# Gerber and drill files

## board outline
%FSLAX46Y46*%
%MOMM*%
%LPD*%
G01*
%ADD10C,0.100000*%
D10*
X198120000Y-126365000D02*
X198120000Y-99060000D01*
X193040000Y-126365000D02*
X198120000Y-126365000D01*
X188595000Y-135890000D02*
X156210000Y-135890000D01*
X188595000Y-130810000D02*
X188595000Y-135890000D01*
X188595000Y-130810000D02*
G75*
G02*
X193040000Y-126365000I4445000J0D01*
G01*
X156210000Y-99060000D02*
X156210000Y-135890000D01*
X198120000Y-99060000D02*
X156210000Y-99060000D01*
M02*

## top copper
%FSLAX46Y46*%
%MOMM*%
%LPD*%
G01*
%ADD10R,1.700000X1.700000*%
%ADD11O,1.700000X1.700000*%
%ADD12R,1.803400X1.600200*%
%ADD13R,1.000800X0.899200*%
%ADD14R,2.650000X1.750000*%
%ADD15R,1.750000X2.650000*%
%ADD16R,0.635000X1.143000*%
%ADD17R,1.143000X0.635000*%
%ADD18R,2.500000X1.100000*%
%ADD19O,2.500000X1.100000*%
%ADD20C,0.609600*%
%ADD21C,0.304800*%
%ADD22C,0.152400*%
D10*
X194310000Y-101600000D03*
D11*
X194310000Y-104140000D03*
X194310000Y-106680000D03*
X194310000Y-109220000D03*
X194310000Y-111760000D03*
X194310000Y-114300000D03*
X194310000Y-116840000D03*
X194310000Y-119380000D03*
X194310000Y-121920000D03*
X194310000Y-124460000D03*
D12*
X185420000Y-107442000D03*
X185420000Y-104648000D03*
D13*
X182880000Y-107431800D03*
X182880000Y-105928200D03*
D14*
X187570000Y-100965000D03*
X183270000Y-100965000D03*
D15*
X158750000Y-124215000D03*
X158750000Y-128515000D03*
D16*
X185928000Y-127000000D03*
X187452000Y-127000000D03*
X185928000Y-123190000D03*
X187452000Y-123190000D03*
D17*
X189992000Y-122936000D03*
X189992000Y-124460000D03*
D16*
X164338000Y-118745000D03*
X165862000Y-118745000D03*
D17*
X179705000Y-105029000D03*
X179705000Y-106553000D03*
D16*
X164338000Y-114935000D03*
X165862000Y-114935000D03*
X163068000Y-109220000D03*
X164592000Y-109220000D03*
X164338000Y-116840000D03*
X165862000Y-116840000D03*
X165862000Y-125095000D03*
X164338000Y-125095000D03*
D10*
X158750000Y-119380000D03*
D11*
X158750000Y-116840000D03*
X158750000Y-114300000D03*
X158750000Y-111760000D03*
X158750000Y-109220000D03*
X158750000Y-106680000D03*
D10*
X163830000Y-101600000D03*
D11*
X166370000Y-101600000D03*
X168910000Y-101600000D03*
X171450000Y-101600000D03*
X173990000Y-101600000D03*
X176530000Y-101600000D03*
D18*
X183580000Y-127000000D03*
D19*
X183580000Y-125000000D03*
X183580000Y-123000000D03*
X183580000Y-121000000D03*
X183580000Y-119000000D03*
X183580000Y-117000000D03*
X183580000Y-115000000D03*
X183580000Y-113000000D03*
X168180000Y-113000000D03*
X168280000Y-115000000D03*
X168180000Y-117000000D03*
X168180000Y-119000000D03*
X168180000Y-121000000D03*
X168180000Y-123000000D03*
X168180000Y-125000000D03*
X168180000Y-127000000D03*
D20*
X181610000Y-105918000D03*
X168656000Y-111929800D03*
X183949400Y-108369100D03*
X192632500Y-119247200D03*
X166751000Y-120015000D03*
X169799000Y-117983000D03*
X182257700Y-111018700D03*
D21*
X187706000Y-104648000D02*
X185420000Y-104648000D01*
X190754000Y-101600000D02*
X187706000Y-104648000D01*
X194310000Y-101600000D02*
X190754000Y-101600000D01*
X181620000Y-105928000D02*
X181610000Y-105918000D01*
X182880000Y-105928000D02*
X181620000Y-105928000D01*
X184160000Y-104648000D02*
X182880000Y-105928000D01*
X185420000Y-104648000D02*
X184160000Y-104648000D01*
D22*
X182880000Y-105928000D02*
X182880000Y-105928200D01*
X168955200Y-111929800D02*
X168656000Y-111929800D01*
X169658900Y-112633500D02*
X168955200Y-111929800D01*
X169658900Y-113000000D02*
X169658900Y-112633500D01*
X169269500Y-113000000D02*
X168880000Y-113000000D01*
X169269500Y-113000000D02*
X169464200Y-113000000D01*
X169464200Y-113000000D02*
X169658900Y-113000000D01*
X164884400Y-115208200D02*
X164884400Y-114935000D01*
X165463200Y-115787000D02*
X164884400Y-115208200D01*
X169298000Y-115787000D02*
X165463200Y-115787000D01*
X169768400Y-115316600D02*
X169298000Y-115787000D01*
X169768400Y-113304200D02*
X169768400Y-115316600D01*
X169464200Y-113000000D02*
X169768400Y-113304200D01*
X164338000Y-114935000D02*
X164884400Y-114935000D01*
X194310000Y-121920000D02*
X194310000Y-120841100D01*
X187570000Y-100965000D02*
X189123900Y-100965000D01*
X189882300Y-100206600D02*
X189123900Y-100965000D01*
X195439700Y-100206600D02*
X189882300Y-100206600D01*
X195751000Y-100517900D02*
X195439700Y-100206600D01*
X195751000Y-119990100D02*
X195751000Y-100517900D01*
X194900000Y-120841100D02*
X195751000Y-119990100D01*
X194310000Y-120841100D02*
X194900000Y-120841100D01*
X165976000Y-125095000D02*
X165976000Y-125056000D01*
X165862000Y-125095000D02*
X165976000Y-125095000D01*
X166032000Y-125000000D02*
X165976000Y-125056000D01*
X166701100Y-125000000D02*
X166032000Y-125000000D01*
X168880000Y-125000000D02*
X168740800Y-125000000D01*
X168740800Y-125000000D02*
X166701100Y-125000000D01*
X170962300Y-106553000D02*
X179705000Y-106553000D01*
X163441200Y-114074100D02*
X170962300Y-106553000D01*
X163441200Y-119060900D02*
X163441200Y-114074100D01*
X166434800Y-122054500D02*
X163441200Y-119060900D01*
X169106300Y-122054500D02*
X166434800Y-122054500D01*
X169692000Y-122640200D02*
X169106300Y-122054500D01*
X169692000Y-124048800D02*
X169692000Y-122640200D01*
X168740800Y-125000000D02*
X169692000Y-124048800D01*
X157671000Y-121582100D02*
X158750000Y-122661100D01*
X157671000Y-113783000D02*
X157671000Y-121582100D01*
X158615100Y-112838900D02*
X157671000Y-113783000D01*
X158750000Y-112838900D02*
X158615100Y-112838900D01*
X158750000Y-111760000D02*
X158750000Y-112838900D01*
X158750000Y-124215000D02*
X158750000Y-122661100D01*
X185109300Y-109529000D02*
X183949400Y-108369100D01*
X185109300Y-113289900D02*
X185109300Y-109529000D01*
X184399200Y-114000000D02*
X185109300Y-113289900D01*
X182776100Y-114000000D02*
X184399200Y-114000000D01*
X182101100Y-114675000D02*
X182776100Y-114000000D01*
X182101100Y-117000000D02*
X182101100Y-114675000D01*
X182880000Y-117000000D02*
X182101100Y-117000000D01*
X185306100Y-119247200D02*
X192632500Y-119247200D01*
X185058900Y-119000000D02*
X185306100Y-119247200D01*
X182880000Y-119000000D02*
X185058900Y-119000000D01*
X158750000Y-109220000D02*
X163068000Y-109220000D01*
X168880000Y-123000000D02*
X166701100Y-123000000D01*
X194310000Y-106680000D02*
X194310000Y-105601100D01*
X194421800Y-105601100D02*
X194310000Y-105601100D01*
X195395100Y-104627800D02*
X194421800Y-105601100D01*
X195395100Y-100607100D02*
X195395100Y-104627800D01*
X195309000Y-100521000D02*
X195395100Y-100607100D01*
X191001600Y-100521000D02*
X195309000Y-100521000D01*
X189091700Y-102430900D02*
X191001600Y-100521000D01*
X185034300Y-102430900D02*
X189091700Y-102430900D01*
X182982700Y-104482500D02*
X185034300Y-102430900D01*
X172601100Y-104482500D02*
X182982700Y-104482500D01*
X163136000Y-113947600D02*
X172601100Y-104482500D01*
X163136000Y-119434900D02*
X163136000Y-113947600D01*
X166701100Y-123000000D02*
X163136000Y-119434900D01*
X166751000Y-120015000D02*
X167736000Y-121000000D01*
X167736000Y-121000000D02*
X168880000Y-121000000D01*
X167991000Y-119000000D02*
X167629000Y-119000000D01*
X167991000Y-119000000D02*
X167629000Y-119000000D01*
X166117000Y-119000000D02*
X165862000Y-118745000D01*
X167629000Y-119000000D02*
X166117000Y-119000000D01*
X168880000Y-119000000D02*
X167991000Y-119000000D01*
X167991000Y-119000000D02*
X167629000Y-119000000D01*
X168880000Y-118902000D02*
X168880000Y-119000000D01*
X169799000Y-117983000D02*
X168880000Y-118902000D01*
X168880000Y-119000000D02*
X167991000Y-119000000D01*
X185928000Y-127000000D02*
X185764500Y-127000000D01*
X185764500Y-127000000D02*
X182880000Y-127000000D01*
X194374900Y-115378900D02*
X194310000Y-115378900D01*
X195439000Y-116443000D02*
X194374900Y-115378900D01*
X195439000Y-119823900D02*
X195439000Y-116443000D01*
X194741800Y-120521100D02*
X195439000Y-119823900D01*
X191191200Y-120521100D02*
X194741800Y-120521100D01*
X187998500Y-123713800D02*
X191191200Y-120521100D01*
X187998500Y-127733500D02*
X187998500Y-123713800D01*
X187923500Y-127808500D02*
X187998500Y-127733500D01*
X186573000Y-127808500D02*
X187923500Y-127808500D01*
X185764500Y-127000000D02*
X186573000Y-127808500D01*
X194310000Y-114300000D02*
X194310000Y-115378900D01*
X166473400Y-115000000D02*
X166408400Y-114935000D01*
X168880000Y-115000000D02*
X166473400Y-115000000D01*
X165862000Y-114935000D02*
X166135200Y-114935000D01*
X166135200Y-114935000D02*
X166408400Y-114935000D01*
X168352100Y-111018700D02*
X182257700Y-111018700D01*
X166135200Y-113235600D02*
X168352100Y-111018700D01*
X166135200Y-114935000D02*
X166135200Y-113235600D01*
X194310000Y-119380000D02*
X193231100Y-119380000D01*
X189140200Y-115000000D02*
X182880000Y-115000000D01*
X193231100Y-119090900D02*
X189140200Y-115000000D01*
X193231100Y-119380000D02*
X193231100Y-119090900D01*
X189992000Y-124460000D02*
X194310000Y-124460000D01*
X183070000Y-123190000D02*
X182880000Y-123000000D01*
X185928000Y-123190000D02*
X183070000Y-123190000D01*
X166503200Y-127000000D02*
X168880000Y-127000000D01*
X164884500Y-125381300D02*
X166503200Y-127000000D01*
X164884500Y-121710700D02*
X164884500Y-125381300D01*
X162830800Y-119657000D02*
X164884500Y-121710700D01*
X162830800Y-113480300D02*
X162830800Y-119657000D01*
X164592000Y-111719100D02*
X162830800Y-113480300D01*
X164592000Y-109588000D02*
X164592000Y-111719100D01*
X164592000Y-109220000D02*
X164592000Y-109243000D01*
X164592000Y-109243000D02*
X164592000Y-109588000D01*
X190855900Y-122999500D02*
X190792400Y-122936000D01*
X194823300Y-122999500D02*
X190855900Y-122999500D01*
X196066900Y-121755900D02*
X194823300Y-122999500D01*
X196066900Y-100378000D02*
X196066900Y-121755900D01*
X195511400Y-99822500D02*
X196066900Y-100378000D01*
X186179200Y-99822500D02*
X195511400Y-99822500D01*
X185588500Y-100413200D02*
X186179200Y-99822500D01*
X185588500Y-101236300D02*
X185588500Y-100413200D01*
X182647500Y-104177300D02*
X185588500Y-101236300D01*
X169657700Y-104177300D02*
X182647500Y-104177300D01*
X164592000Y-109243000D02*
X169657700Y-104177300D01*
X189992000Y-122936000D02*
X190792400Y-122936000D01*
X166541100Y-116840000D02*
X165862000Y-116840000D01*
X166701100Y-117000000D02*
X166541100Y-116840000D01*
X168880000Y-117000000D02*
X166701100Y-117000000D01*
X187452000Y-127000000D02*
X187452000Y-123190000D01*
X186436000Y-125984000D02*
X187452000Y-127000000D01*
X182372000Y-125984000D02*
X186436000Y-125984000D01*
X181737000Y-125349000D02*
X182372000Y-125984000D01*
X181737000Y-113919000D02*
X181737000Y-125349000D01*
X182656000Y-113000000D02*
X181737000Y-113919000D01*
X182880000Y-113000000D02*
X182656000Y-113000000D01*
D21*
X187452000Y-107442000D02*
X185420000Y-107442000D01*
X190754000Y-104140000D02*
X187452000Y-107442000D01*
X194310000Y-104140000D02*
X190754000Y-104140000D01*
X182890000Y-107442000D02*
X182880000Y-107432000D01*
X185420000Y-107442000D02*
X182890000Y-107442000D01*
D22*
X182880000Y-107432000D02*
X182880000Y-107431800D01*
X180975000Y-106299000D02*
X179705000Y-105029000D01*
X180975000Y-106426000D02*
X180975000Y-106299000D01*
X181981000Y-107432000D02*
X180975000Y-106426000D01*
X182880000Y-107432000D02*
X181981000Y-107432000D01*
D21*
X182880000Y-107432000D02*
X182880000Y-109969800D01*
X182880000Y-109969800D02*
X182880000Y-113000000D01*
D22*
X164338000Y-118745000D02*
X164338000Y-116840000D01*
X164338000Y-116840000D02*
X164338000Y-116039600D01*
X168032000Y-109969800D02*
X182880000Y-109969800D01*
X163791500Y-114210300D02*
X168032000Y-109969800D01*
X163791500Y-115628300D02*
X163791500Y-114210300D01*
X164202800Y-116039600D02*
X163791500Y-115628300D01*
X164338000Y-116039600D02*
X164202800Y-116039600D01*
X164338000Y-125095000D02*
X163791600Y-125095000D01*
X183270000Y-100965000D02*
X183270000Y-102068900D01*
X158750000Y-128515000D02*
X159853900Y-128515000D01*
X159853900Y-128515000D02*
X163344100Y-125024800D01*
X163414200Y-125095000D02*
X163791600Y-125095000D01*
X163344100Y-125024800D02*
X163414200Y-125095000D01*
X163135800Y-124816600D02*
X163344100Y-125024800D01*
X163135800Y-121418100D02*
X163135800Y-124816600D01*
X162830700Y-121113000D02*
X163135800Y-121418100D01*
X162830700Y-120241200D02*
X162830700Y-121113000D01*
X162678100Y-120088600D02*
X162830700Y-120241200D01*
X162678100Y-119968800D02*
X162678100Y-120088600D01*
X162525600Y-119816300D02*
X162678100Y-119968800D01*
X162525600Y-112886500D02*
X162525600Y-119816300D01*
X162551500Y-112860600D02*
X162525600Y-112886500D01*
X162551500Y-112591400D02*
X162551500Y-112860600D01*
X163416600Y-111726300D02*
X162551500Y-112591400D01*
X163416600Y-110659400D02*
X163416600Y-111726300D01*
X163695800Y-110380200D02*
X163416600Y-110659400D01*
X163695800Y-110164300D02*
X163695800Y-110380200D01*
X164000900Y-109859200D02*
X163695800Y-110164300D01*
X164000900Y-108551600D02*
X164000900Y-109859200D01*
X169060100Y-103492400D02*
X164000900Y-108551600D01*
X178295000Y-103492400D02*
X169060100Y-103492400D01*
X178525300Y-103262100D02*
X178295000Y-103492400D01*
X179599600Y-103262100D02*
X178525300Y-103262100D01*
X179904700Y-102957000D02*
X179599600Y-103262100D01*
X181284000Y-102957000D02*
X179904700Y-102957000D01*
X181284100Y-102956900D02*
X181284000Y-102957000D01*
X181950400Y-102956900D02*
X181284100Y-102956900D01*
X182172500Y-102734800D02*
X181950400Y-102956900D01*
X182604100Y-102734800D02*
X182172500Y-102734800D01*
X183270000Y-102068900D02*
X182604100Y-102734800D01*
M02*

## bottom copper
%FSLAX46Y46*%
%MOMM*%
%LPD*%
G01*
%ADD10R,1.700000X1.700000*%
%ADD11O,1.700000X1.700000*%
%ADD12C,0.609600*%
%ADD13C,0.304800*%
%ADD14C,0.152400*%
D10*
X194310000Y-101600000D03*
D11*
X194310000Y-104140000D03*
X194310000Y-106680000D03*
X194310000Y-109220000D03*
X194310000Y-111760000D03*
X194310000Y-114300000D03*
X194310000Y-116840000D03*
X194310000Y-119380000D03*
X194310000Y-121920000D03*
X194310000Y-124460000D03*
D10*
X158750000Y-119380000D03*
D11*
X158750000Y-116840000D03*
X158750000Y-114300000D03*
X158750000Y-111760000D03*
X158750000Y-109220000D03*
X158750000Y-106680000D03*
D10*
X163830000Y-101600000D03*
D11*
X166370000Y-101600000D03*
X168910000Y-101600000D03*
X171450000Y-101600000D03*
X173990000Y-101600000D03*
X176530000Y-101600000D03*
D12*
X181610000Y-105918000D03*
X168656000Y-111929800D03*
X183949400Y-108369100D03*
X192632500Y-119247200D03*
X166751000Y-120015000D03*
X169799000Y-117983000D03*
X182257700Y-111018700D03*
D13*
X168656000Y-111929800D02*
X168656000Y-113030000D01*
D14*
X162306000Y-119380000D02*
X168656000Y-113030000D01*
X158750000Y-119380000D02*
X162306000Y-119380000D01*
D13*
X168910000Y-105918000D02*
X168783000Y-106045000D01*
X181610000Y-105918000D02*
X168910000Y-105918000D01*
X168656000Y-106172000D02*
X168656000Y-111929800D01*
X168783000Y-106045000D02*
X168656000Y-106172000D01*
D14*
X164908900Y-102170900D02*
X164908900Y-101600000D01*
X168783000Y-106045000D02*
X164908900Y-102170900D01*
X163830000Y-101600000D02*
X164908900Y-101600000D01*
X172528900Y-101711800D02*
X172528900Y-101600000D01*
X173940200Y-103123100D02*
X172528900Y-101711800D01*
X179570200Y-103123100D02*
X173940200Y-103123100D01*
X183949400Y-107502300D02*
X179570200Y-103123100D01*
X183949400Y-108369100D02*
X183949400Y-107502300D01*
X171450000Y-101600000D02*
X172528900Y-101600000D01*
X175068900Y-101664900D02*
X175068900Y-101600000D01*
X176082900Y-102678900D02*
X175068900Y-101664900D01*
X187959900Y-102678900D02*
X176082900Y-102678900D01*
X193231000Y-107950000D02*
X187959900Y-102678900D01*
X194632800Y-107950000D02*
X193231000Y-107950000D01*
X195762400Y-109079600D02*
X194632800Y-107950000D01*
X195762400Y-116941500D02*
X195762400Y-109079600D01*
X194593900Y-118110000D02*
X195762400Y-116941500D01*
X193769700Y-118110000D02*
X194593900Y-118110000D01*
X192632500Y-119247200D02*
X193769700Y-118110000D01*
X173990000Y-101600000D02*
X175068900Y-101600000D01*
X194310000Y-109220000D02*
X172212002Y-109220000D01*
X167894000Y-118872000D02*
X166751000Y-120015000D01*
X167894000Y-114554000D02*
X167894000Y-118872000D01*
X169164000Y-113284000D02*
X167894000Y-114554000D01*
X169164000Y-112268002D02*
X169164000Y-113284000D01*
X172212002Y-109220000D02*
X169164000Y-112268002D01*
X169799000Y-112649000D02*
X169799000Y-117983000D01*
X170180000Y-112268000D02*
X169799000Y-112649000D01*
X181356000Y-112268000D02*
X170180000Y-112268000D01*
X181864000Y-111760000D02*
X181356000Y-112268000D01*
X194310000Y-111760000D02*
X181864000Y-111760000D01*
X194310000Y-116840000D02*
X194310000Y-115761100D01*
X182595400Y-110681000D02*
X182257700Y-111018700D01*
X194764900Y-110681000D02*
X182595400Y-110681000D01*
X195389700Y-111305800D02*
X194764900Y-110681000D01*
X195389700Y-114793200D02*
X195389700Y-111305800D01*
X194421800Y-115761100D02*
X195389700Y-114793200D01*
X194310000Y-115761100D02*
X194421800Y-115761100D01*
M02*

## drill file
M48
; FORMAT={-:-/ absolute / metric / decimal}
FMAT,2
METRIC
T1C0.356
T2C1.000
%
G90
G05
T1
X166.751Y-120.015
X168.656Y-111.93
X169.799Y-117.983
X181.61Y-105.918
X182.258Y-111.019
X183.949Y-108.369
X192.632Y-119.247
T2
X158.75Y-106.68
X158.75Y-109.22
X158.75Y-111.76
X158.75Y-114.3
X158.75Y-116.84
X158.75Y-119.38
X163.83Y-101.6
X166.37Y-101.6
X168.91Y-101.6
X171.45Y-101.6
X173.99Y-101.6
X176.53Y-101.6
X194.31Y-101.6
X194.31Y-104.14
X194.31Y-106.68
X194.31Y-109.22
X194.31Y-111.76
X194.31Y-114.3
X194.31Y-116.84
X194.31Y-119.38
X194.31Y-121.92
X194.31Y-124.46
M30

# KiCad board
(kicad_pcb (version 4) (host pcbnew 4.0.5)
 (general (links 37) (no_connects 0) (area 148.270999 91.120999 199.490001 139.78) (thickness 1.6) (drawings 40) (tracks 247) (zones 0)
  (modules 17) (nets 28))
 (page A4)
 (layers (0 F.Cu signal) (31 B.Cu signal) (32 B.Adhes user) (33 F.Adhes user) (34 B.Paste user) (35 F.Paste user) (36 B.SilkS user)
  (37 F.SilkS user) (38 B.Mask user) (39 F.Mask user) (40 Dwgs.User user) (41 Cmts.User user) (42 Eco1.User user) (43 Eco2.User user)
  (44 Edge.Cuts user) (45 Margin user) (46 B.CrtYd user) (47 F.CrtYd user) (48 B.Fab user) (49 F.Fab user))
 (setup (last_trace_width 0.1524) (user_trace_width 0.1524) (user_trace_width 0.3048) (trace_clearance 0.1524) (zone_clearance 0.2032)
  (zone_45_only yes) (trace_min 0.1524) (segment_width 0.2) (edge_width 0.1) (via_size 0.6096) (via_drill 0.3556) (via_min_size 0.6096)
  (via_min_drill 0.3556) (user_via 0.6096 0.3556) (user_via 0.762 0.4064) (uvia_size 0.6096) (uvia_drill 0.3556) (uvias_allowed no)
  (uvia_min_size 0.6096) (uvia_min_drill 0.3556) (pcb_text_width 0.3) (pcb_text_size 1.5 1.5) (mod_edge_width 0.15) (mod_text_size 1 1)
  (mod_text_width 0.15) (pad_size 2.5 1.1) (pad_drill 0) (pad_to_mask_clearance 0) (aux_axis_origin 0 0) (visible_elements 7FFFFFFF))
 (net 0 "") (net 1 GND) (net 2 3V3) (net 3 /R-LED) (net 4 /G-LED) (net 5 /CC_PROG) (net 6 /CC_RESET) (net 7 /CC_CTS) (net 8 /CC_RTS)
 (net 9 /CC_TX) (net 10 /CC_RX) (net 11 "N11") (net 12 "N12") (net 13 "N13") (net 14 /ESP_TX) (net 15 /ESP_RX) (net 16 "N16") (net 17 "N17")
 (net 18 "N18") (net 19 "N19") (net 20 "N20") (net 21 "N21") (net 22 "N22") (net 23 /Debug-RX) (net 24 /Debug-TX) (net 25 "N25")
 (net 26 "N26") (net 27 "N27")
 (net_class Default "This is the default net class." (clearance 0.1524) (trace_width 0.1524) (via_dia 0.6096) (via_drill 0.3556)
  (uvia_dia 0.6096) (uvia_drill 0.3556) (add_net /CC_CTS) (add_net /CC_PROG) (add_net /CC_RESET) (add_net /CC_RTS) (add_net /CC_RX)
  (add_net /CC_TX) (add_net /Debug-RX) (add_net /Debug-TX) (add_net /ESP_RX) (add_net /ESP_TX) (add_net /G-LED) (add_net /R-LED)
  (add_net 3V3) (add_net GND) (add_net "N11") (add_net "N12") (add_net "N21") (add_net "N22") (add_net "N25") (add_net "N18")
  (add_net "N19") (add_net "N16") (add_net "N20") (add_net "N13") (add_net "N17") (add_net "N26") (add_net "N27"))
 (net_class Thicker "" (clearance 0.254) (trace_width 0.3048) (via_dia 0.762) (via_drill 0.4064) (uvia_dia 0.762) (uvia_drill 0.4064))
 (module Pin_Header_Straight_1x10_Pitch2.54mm (layer B.Cu) (at 194.31 101.6 180)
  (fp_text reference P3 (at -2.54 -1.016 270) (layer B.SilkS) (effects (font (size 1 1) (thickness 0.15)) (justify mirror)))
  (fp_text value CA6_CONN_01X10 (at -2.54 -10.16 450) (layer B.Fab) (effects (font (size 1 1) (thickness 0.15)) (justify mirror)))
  (pad 1 thru_hole rect (at 0 0 180) (size 1.7 1.7) (drill 1) (layers *.Cu *.Mask) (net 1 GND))
  (pad 2 thru_hole oval (at 0 -2.54 180) (size 1.7 1.7) (drill 1) (layers *.Cu *.Mask) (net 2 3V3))
  (pad 3 thru_hole oval (at 0 -5.08 180) (size 1.7 1.7) (drill 1) (layers *.Cu *.Mask) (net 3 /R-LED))
  (pad 4 thru_hole oval (at 0 -7.62 180) (size 1.7 1.7) (drill 1) (layers *.Cu *.Mask) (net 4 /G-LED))
  (pad 5 thru_hole oval (at 0 -10.16 180) (size 1.7 1.7) (drill 1) (layers *.Cu *.Mask) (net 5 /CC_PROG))
  (pad 6 thru_hole oval (at 0 -12.7 180) (size 1.7 1.7) (drill 1) (layers *.Cu *.Mask) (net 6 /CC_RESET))
  (pad 7 thru_hole oval (at 0 -15.24 180) (size 1.7 1.7) (drill 1) (layers *.Cu *.Mask) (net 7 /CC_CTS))
  (pad 8 thru_hole oval (at 0 -17.78 180) (size 1.7 1.7) (drill 1) (layers *.Cu *.Mask) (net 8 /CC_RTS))
  (pad 9 thru_hole oval (at 0 -20.32 180) (size 1.7 1.7) (drill 1) (layers *.Cu *.Mask) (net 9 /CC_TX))
  (pad 10 thru_hole oval (at 0 -22.86 180) (size 1.7 1.7) (drill 1) (layers *.Cu *.Mask) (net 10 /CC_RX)))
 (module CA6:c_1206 (layer F.Cu) (at 185.42 106.045 270)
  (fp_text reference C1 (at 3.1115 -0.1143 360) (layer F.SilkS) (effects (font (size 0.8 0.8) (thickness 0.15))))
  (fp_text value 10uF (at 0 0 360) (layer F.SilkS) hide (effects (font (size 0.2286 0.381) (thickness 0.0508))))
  (pad 1 smd rect (at 1.397 0 270) (size 1.6002 1.8034) (layers F.Cu F.Paste F.Mask) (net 2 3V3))
  (pad 2 smd rect (at -1.397 0 270) (size 1.6002 1.8034) (layers F.Cu F.Paste F.Mask) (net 1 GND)))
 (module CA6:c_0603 (layer F.Cu) (at 182.88 106.68 270)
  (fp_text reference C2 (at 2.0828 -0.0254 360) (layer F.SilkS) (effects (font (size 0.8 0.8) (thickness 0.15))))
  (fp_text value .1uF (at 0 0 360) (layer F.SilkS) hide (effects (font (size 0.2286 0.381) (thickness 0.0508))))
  (pad 1 smd rect (at 0.7518 0 270) (size 0.8992 1.0008) (layers F.Cu F.Paste F.Mask) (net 2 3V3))
  (pad 2 smd rect (at -0.7518 0 270) (size 0.8992 1.0008) (layers F.Cu F.Paste F.Mask) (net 1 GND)))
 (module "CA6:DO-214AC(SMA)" (layer F.Cu) (at 185.42 100.965 180)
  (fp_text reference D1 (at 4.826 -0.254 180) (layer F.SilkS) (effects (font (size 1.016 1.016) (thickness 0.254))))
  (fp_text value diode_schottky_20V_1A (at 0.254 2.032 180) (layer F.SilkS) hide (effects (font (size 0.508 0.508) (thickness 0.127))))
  (pad 1 smd rect (at -2.15 0 180) (size 2.65 1.75) (layers F.Cu F.Paste F.Mask) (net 9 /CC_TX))
  (pad 2 smd rect (at 2.15 0 180) (size 2.65 1.75) (layers F.Cu F.Paste F.Mask) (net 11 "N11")))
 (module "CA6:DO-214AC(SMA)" (layer F.Cu) (at 158.75 126.365 270)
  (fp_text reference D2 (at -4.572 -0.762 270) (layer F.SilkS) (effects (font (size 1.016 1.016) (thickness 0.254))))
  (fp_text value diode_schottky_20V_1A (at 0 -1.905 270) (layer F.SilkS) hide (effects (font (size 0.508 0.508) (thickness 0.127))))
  (pad 1 smd rect (at -2.15 0 270) (size 2.65 1.75) (layers F.Cu F.Paste F.Mask) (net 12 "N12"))
  (pad 2 smd rect (at 2.15 0 270) (size 2.65 1.75) (layers F.Cu F.Paste F.Mask) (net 11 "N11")))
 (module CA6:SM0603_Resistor (layer F.Cu) (at 186.69 127)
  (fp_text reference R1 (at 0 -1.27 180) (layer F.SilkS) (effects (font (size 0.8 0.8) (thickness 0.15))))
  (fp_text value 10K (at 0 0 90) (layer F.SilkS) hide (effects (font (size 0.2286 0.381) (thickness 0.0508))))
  (pad 1 smd rect (at -0.762 0) (size 0.635 1.143) (layers F.Cu F.Paste F.Mask) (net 6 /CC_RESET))
  (pad 2 smd rect (at 0.762 0) (size 0.635 1.143) (layers F.Cu F.Paste F.Mask) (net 2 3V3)))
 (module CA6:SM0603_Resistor (layer F.Cu) (at 186.69 123.19)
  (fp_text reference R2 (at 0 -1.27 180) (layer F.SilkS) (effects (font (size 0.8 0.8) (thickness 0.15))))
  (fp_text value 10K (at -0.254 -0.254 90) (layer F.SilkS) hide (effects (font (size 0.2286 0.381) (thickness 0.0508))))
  (pad 1 smd rect (at -0.762 0) (size 0.635 1.143) (layers F.Cu F.Paste F.Mask) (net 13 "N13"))
  (pad 2 smd rect (at 0.762 0) (size 0.635 1.143) (layers F.Cu F.Paste F.Mask) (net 2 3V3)))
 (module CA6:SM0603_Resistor (layer F.Cu) (at 189.992 123.698 270)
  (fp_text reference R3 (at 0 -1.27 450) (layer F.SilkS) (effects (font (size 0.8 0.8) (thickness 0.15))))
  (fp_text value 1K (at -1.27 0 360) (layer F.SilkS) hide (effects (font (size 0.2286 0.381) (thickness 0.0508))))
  (pad 1 smd rect (at -0.762 0 270) (size 0.635 1.143) (layers F.Cu F.Paste F.Mask) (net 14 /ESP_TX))
  (pad 2 smd rect (at 0.762 0 270) (size 0.635 1.143) (layers F.Cu F.Paste F.Mask) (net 10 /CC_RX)))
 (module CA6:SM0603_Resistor (layer F.Cu) (at 165.1 118.745)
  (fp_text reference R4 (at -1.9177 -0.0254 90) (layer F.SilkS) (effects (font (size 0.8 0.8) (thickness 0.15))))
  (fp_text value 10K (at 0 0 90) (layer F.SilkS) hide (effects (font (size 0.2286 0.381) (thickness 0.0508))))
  (pad 1 smd rect (at -0.762 0) (size 0.635 1.143) (layers F.Cu F.Paste F.Mask) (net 2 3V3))
  (pad 2 smd rect (at 0.762 0) (size 0.635 1.143) (layers F.Cu F.Paste F.Mask) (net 5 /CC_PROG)))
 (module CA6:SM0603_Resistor (layer F.Cu) (at 179.705 105.791 270)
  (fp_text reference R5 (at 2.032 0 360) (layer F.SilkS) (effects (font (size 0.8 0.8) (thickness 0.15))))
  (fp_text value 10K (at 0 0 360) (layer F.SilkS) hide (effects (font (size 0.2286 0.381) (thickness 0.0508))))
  (pad 1 smd rect (at -0.762 0 270) (size 0.635 1.143) (layers F.Cu F.Paste F.Mask) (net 2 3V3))
  (pad 2 smd rect (at 0.762 0 270) (size 0.635 1.143) (layers F.Cu F.Paste F.Mask) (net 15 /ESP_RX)))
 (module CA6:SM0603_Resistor (layer F.Cu) (at 165.1 114.935)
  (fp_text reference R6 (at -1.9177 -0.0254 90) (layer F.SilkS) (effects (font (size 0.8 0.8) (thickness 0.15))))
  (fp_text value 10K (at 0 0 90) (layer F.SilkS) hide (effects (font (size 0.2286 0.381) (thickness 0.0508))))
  (pad 1 smd rect (at -0.762 0) (size 0.635 1.143) (layers F.Cu F.Paste F.Mask) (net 1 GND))
  (pad 2 smd rect (at 0.762 0) (size 0.635 1.143) (layers F.Cu F.Paste F.Mask) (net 7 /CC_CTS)))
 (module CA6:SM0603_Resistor (layer F.Cu) (at 163.83 109.22)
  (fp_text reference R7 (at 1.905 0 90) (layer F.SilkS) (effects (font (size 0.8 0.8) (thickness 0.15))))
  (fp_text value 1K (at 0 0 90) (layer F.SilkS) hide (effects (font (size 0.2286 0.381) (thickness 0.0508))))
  (pad 1 smd rect (at -0.762 0) (size 0.635 1.143) (layers F.Cu F.Paste F.Mask) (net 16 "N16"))
  (pad 2 smd rect (at 0.762 0) (size 0.635 1.143) (layers F.Cu F.Paste F.Mask) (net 14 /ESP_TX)))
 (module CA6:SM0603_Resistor (layer F.Cu) (at 165.1 116.84)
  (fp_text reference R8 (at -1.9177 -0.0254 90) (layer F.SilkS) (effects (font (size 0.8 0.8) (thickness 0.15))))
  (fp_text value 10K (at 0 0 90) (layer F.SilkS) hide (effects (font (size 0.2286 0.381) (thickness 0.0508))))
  (pad 1 smd rect (at -0.762 0) (size 0.635 1.143) (layers F.Cu F.Paste F.Mask) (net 2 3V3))
  (pad 2 smd rect (at 0.762 0) (size 0.635 1.143) (layers F.Cu F.Paste F.Mask) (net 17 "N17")))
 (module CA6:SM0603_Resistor (layer F.Cu) (at 165.1 125.095 180)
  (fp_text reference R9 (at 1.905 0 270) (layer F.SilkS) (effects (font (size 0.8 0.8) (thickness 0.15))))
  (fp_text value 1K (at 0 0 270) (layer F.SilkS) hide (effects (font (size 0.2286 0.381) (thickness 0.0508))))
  (pad 1 smd rect (at -0.762 0 180) (size 0.635 1.143) (layers F.Cu F.Paste F.Mask) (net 15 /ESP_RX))
  (pad 2 smd rect (at 0.762 0 180) (size 0.635 1.143) (layers F.Cu F.Paste F.Mask) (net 11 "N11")))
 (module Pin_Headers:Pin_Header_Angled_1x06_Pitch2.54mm (layer F.Cu) (at 158.75 119.38 180)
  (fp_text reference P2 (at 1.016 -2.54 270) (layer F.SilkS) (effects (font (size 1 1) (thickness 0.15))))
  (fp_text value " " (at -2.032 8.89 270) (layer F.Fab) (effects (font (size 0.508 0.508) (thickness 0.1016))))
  (pad 1 thru_hole rect (at 0 0 180) (size 1.7 1.7) (drill 1) (layers *.Cu *.Mask) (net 1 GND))
  (pad 2 thru_hole oval (at 0 2.54 180) (size 1.7 1.7) (drill 1) (layers *.Cu *.Mask) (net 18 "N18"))
  (pad 3 thru_hole oval (at 0 5.08 180) (size 1.7 1.7) (drill 1) (layers *.Cu *.Mask) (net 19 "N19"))
  (pad 4 thru_hole oval (at 0 7.62 180) (size 1.7 1.7) (drill 1) (layers *.Cu *.Mask) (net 12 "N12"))
  (pad 5 thru_hole oval (at 0 10.16 180) (size 1.7 1.7) (drill 1) (layers *.Cu *.Mask) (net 16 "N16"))
  (pad 6 thru_hole oval (at 0 12.7 180) (size 1.7 1.7) (drill 1) (layers *.Cu *.Mask) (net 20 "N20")))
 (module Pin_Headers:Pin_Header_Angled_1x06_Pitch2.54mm (layer F.Cu) (at 163.83 101.6 90)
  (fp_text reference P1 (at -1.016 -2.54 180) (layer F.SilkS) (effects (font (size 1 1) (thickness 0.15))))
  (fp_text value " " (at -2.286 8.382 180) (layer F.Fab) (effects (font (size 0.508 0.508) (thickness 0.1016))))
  (pad 1 thru_hole rect (at 0 0 90) (size 1.7 1.7) (drill 1) (layers *.Cu *.Mask) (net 1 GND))
  (pad 2 thru_hole oval (at 0 2.54 90) (size 1.7 1.7) (drill 1) (layers *.Cu *.Mask) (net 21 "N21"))
  (pad 3 thru_hole oval (at 0 5.08 90) (size 1.7 1.7) (drill 1) (layers *.Cu *.Mask) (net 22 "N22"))
  (pad 4 thru_hole oval (at 0 7.62 90) (size 1.7 1.7) (drill 1) (layers *.Cu *.Mask) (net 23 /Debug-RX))
  (pad 5 thru_hole oval (at 0 10.16 90) (size 1.7 1.7) (drill 1) (layers *.Cu *.Mask) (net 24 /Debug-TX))
  (pad 6 thru_hole oval (at 0 12.7 90) (size 1.7 1.7) (drill 1) (layers *.Cu *.Mask) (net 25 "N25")))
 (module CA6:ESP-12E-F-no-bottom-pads (layer F.Cu) (at 182.88 127 180)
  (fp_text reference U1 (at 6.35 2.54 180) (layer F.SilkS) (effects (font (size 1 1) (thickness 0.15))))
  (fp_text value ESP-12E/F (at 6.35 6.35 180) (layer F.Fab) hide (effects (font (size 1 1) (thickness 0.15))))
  (pad 1 smd rect (at 0 0 180) (size 2.5 1.1) (drill (offset -0.7 0)) (layers F.Cu F.Paste F.Mask) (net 6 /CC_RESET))
  (pad 2 smd oval (at 0 2 180) (size 2.5 1.1) (drill (offset -0.7 0)) (layers F.Cu F.Paste F.Mask) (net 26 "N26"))
  (pad 3 smd oval (at 0 4 180) (size 2.5 1.1) (drill (offset -0.7 0)) (layers F.Cu F.Paste F.Mask) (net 13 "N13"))
  (pad 4 smd oval (at 0 6 180) (size 2.5 1.1) (drill (offset -0.7 0)) (layers F.Cu F.Paste F.Mask) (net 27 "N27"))
  (pad 5 smd oval (at 0 8 180) (size 2.5 1.1) (drill (offset -0.7 0)) (layers F.Cu F.Paste F.Mask) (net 24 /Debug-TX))
  (pad 6 smd oval (at 0 10 180) (size 2.5 1.1) (drill (offset -0.7 0)) (layers F.Cu F.Paste F.Mask) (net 23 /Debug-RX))
  (pad 7 smd oval (at 0 12 180) (size 2.5 1.1) (drill (offset -0.7 0)) (layers F.Cu F.Paste F.Mask) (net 8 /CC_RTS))
  (pad 8 smd oval (at 0 14 180) (size 2.5 1.1) (drill (offset -0.7 0)) (layers F.Cu F.Paste F.Mask) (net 2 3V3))
  (pad 9 smd oval (at 14 14 180) (size 2.5 1.1) (drill (offset 0.7 0)) (layers F.Cu F.Paste F.Mask) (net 1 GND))
  (pad 10 smd oval (at 14 12 180) (size 2.5 1.1) (drill (offset 0.6 0)) (layers F.Cu F.Paste F.Mask) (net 7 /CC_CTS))
  (pad 11 smd oval (at 14 10 180) (size 2.5 1.1) (drill (offset 0.7 0)) (layers F.Cu F.Paste F.Mask) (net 17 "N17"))
  (pad 12 smd oval (at 14 8 180) (size 2.5 1.1) (drill (offset 0.7 0)) (layers F.Cu F.Paste F.Mask) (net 5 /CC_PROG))
  (pad 13 smd oval (at 14 6 180) (size 2.5 1.1) (drill (offset 0.7 0)) (layers F.Cu F.Paste F.Mask) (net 4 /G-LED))
  (pad 14 smd oval (at 14 4 180) (size 2.5 1.1) (drill (offset 0.7 0)) (layers F.Cu F.Paste F.Mask) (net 3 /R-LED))
  (pad 15 smd oval (at 14 2 180) (size 2.5 1.1) (drill (offset 0.7 0)) (layers F.Cu F.Paste F.Mask) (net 15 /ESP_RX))
  (pad 16 smd oval (at 14 0 180) (size 2.5 1.1) (drill (offset 0.7 0)) (layers F.Cu F.Paste F.Mask) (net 14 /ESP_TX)))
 (gr_line (start 198.12 126.365) (end 198.12 99.06) (angle 90) (layer Edge.Cuts) (width 0.1))
 (gr_line (start 193.04 126.365) (end 198.12 126.365) (angle 90) (layer Edge.Cuts) (width 0.1))
 (gr_line (start 188.595 135.89) (end 156.21 135.89) (angle 90) (layer Edge.Cuts) (width 0.1))
 (gr_line (start 188.595 130.81) (end 188.595 135.89) (angle 90) (layer Edge.Cuts) (width 0.1))
 (gr_arc (start 193.04 130.81) (end 188.595 130.81) (angle 90) (layer Edge.Cuts) (width 0.1))
 (gr_line (start 156.21 99.06) (end 156.21 135.89) (angle 90) (layer Edge.Cuts) (width 0.1))
 (gr_line (start 198.12 99.06) (end 156.21 99.06) (angle 90) (layer Edge.Cuts) (width 0.1))
 (via (at 181.61 105.918) (size 0.6096) (layers F.Cu B.Cu) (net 1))
 (via (at 168.656 111.9298) (size 0.6096) (layers F.Cu B.Cu) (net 1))
 (segment (start 187.706 104.648) (end 185.42 104.648) (width 0.3048) (layer F.Cu) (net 1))
 (segment (start 190.754 101.6) (end 187.706 104.648) (width 0.3048) (layer F.Cu) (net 1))
 (segment (start 194.31 101.6) (end 190.754 101.6) (width 0.3048) (layer F.Cu) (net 1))
 (segment (start 181.62 105.928) (end 181.61 105.918) (width 0.3048) (layer F.Cu) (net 1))
 (segment (start 182.88 105.928) (end 181.62 105.928) (width 0.3048) (layer F.Cu) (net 1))
 (segment (start 184.16 104.648) (end 182.88 105.928) (width 0.3048) (layer F.Cu) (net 1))
 (segment (start 185.42 104.648) (end 184.16 104.648) (width 0.3048) (layer F.Cu) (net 1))
 (segment (start 182.88 105.928) (end 182.88 105.9282) (width 0.1524) (layer F.Cu) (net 1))
 (segment (start 168.656 111.9298) (end 168.656 113.03) (width 0.3048) (layer B.Cu) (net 1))
 (segment (start 168.9552 111.9298) (end 168.656 111.9298) (width 0.1524) (layer F.Cu) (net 1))
 (segment (start 169.6589 112.6335) (end 168.9552 111.9298) (width 0.1524) (layer F.Cu) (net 1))
 (segment (start 169.6589 113) (end 169.6589 112.6335) (width 0.1524) (layer F.Cu) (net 1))
 (segment (start 169.2695 113) (end 168.88 113) (width 0.1524) (layer F.Cu) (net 1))
 (segment (start 162.306 119.38) (end 168.656 113.03) (width 0.1524) (layer B.Cu) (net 1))
 (segment (start 158.75 119.38) (end 162.306 119.38) (width 0.1524) (layer B.Cu) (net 1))
 (segment (start 169.2695 113) (end 169.4642 113) (width 0.1524) (layer F.Cu) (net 1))
 (segment (start 169.4642 113) (end 169.6589 113) (width 0.1524) (layer F.Cu) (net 1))
 (segment (start 164.8844 115.2082) (end 164.8844 114.935) (width 0.1524) (layer F.Cu) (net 1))
 (segment (start 165.4632 115.787) (end 164.8844 115.2082) (width 0.1524) (layer F.Cu) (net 1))
 (segment (start 169.298 115.787) (end 165.4632 115.787) (width 0.1524) (layer F.Cu) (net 1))
 (segment (start 169.7684 115.3166) (end 169.298 115.787) (width 0.1524) (layer F.Cu) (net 1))
 (segment (start 169.7684 113.3042) (end 169.7684 115.3166) (width 0.1524) (layer F.Cu) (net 1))
 (segment (start 169.4642 113) (end 169.7684 113.3042) (width 0.1524) (layer F.Cu) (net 1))
 (segment (start 164.338 114.935) (end 164.8844 114.935) (width 0.1524) (layer F.Cu) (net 1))
 (segment (start 168.91 105.918) (end 168.783 106.045) (width 0.3048) (layer B.Cu) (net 1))
 (segment (start 181.61 105.918) (end 168.91 105.918) (width 0.3048) (layer B.Cu) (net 1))
 (segment (start 168.656 106.172) (end 168.656 111.9298) (width 0.3048) (layer B.Cu) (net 1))
 (segment (start 168.783 106.045) (end 168.656 106.172) (width 0.3048) (layer B.Cu) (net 1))
 (segment (start 164.9089 102.1709) (end 164.9089 101.6) (width 0.1524) (layer B.Cu) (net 1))
 (segment (start 168.783 106.045) (end 164.9089 102.1709) (width 0.1524) (layer B.Cu) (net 1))
 (segment (start 163.83 101.6) (end 164.9089 101.6) (width 0.1524) (layer B.Cu) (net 1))
 (segment (start 194.31 121.92) (end 194.31 120.8411) (width 0.1524) (layer F.Cu) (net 9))
 (segment (start 187.57 100.965) (end 189.1239 100.965) (width 0.1524) (layer F.Cu) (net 9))
 (segment (start 189.8823 100.2066) (end 189.1239 100.965) (width 0.1524) (layer F.Cu) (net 9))
 (segment (start 195.4397 100.2066) (end 189.8823 100.2066) (width 0.1524) (layer F.Cu) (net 9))
 (segment (start 195.751 100.5179) (end 195.4397 100.2066) (width 0.1524) (layer F.Cu) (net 9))
 (segment (start 195.751 119.9901) (end 195.751 100.5179) (width 0.1524) (layer F.Cu) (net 9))
 (segment (start 194.9 120.8411) (end 195.751 119.9901) (width 0.1524) (layer F.Cu) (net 9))
 (segment (start 194.31 120.8411) (end 194.9 120.8411) (width 0.1524) (layer F.Cu) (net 9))
 (segment (start 165.976 125.095) (end 165.976 125.056) (width 0.1524) (layer F.Cu) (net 15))
 (segment (start 165.862 125.095) (end 165.976 125.095) (width 0.1524) (layer F.Cu) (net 15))
 (segment (start 166.032 125) (end 165.976 125.056) (width 0.1524) (layer F.Cu) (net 15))
 (segment (start 166.7011 125) (end 166.032 125) (width 0.1524) (layer F.Cu) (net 15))
 (segment (start 168.88 125) (end 168.7408 125) (width 0.1524) (layer F.Cu) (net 15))
 (segment (start 168.7408 125) (end 166.7011 125) (width 0.1524) (layer F.Cu) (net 15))
 (segment (start 170.9623 106.553) (end 179.705 106.553) (width 0.1524) (layer F.Cu) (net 15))
 (segment (start 163.4412 114.0741) (end 170.9623 106.553) (width 0.1524) (layer F.Cu) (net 15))
 (segment (start 163.4412 119.0609) (end 163.4412 114.0741) (width 0.1524) (layer F.Cu) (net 15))
 (segment (start 166.4348 122.0545) (end 163.4412 119.0609) (width 0.1524) (layer F.Cu) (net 15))
 (segment (start 169.1063 122.0545) (end 166.4348 122.0545) (width 0.1524) (layer F.Cu) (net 15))
 (segment (start 169.692 122.6402) (end 169.1063 122.0545) (width 0.1524) (layer F.Cu) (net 15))
 (segment (start 169.692 124.0488) (end 169.692 122.6402) (width 0.1524) (layer F.Cu) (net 15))
 (segment (start 168.7408 125) (end 169.692 124.0488) (width 0.1524) (layer F.Cu) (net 15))
 (segment (start 157.671 121.5821) (end 158.75 122.6611) (width 0.1524) (layer F.Cu) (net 12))
 (segment (start 157.671 113.783) (end 157.671 121.5821) (width 0.1524) (layer F.Cu) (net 12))
 (segment (start 158.6151 112.8389) (end 157.671 113.783) (width 0.1524) (layer F.Cu) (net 12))
 (segment (start 158.75 112.8389) (end 158.6151 112.8389) (width 0.1524) (layer F.Cu) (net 12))
 (segment (start 158.75 111.76) (end 158.75 112.8389) (width 0.1524) (layer F.Cu) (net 12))
 (segment (start 158.75 124.215) (end 158.75 122.6611) (width 0.1524) (layer F.Cu) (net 12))
 (via (at 183.9494 108.3691) (size 0.6096) (layers F.Cu B.Cu) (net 23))
 (segment (start 185.1093 109.529) (end 183.9494 108.3691) (width 0.1524) (layer F.Cu) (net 23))
 (segment (start 185.1093 113.2899) (end 185.1093 109.529) (width 0.1524) (layer F.Cu) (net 23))
 (segment (start 184.3992 114) (end 185.1093 113.2899) (width 0.1524) (layer F.Cu) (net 23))
 (segment (start 182.7761 114) (end 184.3992 114) (width 0.1524) (layer F.Cu) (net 23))
 (segment (start 182.1011 114.675) (end 182.7761 114) (width 0.1524) (layer F.Cu) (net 23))
 (segment (start 182.1011 117) (end 182.1011 114.675) (width 0.1524) (layer F.Cu) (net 23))
 (segment (start 172.5289 101.7118) (end 172.5289 101.6) (width 0.1524) (layer B.Cu) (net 23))
 (segment (start 173.9402 103.1231) (end 172.5289 101.7118) (width 0.1524) (layer B.Cu) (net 23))
 (segment (start 179.5702 103.1231) (end 173.9402 103.1231) (width 0.1524) (layer B.Cu) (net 23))
 (segment (start 183.9494 107.5023) (end 179.5702 103.1231) (width 0.1524) (layer B.Cu) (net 23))
 (segment (start 183.9494 108.3691) (end 183.9494 107.5023) (width 0.1524) (layer B.Cu) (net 23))
 (segment (start 182.88 117) (end 182.1011 117) (width 0.1524) (layer F.Cu) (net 23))
 (segment (start 171.45 101.6) (end 172.5289 101.6) (width 0.1524) (layer B.Cu) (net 23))
 (via (at 192.6325 119.2472) (size 0.6096) (layers F.Cu B.Cu) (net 24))
 (segment (start 185.3061 119.2472) (end 192.6325 119.2472) (width 0.1524) (layer F.Cu) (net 24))
 (segment (start 185.0589 119) (end 185.3061 119.2472) (width 0.1524) (layer F.Cu) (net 24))
 (segment (start 175.0689 101.6649) (end 175.0689 101.6) (width 0.1524) (layer B.Cu) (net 24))
 (segment (start 176.0829 102.6789) (end 175.0689 101.6649) (width 0.1524) (layer B.Cu) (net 24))
 (segment (start 187.9599 102.6789) (end 176.0829 102.6789) (width 0.1524) (layer B.Cu) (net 24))
 (segment (start 193.231 107.95) (end 187.9599 102.6789) (width 0.1524) (layer B.Cu) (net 24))
 (segment (start 194.6328 107.95) (end 193.231 107.95) (width 0.1524) (layer B.Cu) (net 24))
 (segment (start 195.7624 109.0796) (end 194.6328 107.95) (width 0.1524) (layer B.Cu) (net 24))
 (segment (start 195.7624 116.9415) (end 195.7624 109.0796) (width 0.1524) (layer B.Cu) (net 24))
 (segment (start 194.5939 118.11) (end 195.7624 116.9415) (width 0.1524) (layer B.Cu) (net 24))
 (segment (start 193.7697 118.11) (end 194.5939 118.11) (width 0.1524) (layer B.Cu) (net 24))
 (segment (start 192.6325 119.2472) (end 193.7697 118.11) (width 0.1524) (layer B.Cu) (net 24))
 (segment (start 182.88 119) (end 185.0589 119) (width 0.1524) (layer F.Cu) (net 24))
 (segment (start 173.99 101.6) (end 175.0689 101.6) (width 0.1524) (layer B.Cu) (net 24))
 (segment (start 158.75 109.22) (end 163.068 109.22) (width 0.1524) (layer F.Cu) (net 16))
 (segment (start 168.88 123) (end 166.7011 123) (width 0.1524) (layer F.Cu) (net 3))
 (segment (start 194.31 106.68) (end 194.31 105.6011) (width 0.1524) (layer F.Cu) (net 3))
 (segment (start 194.4218 105.6011) (end 194.31 105.6011) (width 0.1524) (layer F.Cu) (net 3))
 (segment (start 195.3951 104.6278) (end 194.4218 105.6011) (width 0.1524) (layer F.Cu) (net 3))
 (segment (start 195.3951 100.6071) (end 195.3951 104.6278) (width 0.1524) (layer F.Cu) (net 3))
 (segment (start 195.309 100.521) (end 195.3951 100.6071) (width 0.1524) (layer F.Cu) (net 3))
 (segment (start 191.0016 100.521) (end 195.309 100.521) (width 0.1524) (layer F.Cu) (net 3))
 (segment (start 189.0917 102.4309) (end 191.0016 100.521) (width 0.1524) (layer F.Cu) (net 3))
 (segment (start 185.0343 102.4309) (end 189.0917 102.4309) (width 0.1524) (layer F.Cu) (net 3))
 (segment (start 182.9827 104.4825) (end 185.0343 102.4309) (width 0.1524) (layer F.Cu) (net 3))
 (segment (start 172.6011 104.4825) (end 182.9827 104.4825) (width 0.1524) (layer F.Cu) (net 3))
 (segment (start 163.136 113.9476) (end 172.6011 104.4825) (width 0.1524) (layer F.Cu) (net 3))
 (segment (start 163.136 119.4349) (end 163.136 113.9476) (width 0.1524) (layer F.Cu) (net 3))
 (segment (start 166.7011 123) (end 163.136 119.4349) (width 0.1524) (layer F.Cu) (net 3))
 (segment (start 194.31 109.22) (end 172.212002 109.22) (width 0.1524) (layer B.Cu) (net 4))
 (segment (start 166.751 120.015) (end 167.736 121) (width 0.1524) (layer F.Cu) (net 4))
 (via (at 166.751 120.015) (size 0.6096) (drill 0.3556) (layers F.Cu B.Cu) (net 4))
 (segment (start 167.894 118.872) (end 166.751 120.015) (width 0.1524) (layer B.Cu) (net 4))
 (segment (start 167.894 114.554) (end 167.894 118.872) (width 0.1524) (layer B.Cu) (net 4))
 (segment (start 169.164 113.284) (end 167.894 114.554) (width 0.1524) (layer B.Cu) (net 4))
 (segment (start 169.164 112.268002) (end 169.164 113.284) (width 0.1524) (layer B.Cu) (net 4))
 (segment (start 172.212002 109.22) (end 169.164 112.268002) (width 0.1524) (layer B.Cu) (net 4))
 (segment (start 167.736 121) (end 168.88 121) (width 0.1524) (layer F.Cu) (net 4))
 (via (at 169.799 117.983) (size 0.6096) (layers F.Cu B.Cu) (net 5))
 (segment (start 169.799 112.649) (end 169.799 117.983) (width 0.1524) (layer B.Cu) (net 5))
 (segment (start 170.18 112.268) (end 169.799 112.649) (width 0.1524) (layer B.Cu) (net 5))
 (segment (start 181.356 112.268) (end 170.18 112.268) (width 0.1524) (layer B.Cu) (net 5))
 (segment (start 181.864 111.76) (end 181.356 112.268) (width 0.1524) (layer B.Cu) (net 5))
 (segment (start 194.31 111.76) (end 181.864 111.76) (width 0.1524) (layer B.Cu) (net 5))
 (segment (start 167.991 119) (end 167.629 119) (width 0.1524) (layer F.Cu) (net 5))
 (segment (start 167.991 119) (end 167.629 119) (width 0.1524) (layer F.Cu) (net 5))
 (segment (start 166.117 119) (end 165.862 118.745) (width 0.1524) (layer F.Cu) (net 5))
 (segment (start 167.629 119) (end 166.117 119) (width 0.1524) (layer F.Cu) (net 5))
 (segment (start 168.88 119) (end 167.991 119) (width 0.1524) (layer F.Cu) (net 5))
 (segment (start 167.991 119) (end 167.629 119) (width 0.1524) (layer F.Cu) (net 5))
 (segment (start 168.88 118.902) (end 168.88 119) (width 0.1524) (layer F.Cu) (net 5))
 (segment (start 169.799 117.983) (end 168.88 118.902) (width 0.1524) (layer F.Cu) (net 5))
 (segment (start 168.88 119) (end 167.991 119) (width 0.1524) (layer F.Cu) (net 5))
 (segment (start 185.928 127) (end 185.7645 127) (width 0.1524) (layer F.Cu) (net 6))
 (segment (start 185.7645 127) (end 182.88 127) (width 0.1524) (layer F.Cu) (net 6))
 (segment (start 194.3749 115.3789) (end 194.31 115.3789) (width 0.1524) (layer F.Cu) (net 6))
 (segment (start 195.439 116.443) (end 194.3749 115.3789) (width 0.1524) (layer F.Cu) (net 6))
 (segment (start 195.439 119.8239) (end 195.439 116.443) (width 0.1524) (layer F.Cu) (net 6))
 (segment (start 194.7418 120.5211) (end 195.439 119.8239) (width 0.1524) (layer F.Cu) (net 6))
 (segment (start 191.1912 120.5211) (end 194.7418 120.5211) (width 0.1524) (layer F.Cu) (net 6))
 (segment (start 187.9985 123.7138) (end 191.1912 120.5211) (width 0.1524) (layer F.Cu) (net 6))
 (segment (start 187.9985 127.7335) (end 187.9985 123.7138) (width 0.1524) (layer F.Cu) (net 6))
 (segment (start 187.9235 127.8085) (end 187.9985 127.7335) (width 0.1524) (layer F.Cu) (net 6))
 (segment (start 186.573 127.8085) (end 187.9235 127.8085) (width 0.1524) (layer F.Cu) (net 6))
 (segment (start 185.7645 127) (end 186.573 127.8085) (width 0.1524) (layer F.Cu) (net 6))
 (segment (start 194.31 114.3) (end 194.31 115.3789) (width 0.1524) (layer F.Cu) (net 6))
 (via (at 182.2577 111.0187) (size 0.6096) (layers F.Cu B.Cu) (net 7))
 (segment (start 166.4734 115) (end 166.4084 114.935) (width 0.1524) (layer F.Cu) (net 7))
 (segment (start 168.88 115) (end 166.4734 115) (width 0.1524) (layer F.Cu) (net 7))
 (segment (start 165.862 114.935) (end 166.1352 114.935) (width 0.1524) (layer F.Cu) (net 7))
 (segment (start 166.1352 114.935) (end 166.4084 114.935) (width 0.1524) (layer F.Cu) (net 7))
 (segment (start 194.31 116.84) (end 194.31 115.7611) (width 0.1524) (layer B.Cu) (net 7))
 (segment (start 182.5954 110.681) (end 182.2577 111.0187) (width 0.1524) (layer B.Cu) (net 7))
 (segment (start 194.7649 110.681) (end 182.5954 110.681) (width 0.1524) (layer B.Cu) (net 7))
 (segment (start 195.3897 111.3058) (end 194.7649 110.681) (width 0.1524) (layer B.Cu) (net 7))
 (segment (start 195.3897 114.7932) (end 195.3897 111.3058) (width 0.1524) (layer B.Cu) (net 7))
 (segment (start 194.4218 115.7611) (end 195.3897 114.7932) (width 0.1524) (layer B.Cu) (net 7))
 (segment (start 194.31 115.7611) (end 194.4218 115.7611) (width 0.1524) (layer B.Cu) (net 7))
 (segment (start 168.3521 111.0187) (end 182.2577 111.0187) (width 0.1524) (layer F.Cu) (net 7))
 (segment (start 166.1352 113.2356) (end 168.3521 111.0187) (width 0.1524) (layer F.Cu) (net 7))
 (segment (start 166.1352 114.935) (end 166.1352 113.2356) (width 0.1524) (layer F.Cu) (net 7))
 (segment (start 194.31 119.38) (end 193.2311 119.38) (width 0.1524) (layer F.Cu) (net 8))
 (segment (start 189.1402 115) (end 182.88 115) (width 0.1524) (layer F.Cu) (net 8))
 (segment (start 193.2311 119.0909) (end 189.1402 115) (width 0.1524) (layer F.Cu) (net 8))
 (segment (start 193.2311 119.38) (end 193.2311 119.0909) (width 0.1524) (layer F.Cu) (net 8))
 (segment (start 189.992 124.46) (end 194.31 124.46) (width 0.1524) (layer F.Cu) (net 10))
 (segment (start 183.07 123.19) (end 182.88 123) (width 0.1524) (layer F.Cu) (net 13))
 (segment (start 185.928 123.19) (end 183.07 123.19) (width 0.1524) (layer F.Cu) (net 13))
 (segment (start 166.5032 127) (end 168.88 127) (width 0.1524) (layer F.Cu) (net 14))
 (segment (start 164.8845 125.3813) (end 166.5032 127) (width 0.1524) (layer F.Cu) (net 14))
 (segment (start 164.8845 121.7107) (end 164.8845 125.3813) (width 0.1524) (layer F.Cu) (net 14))
 (segment (start 162.8308 119.657) (end 164.8845 121.7107) (width 0.1524) (layer F.Cu) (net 14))
 (segment (start 162.8308 113.4803) (end 162.8308 119.657) (width 0.1524) (layer F.Cu) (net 14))
 (segment (start 164.592 111.7191) (end 162.8308 113.4803) (width 0.1524) (layer F.Cu) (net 14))
 (segment (start 164.592 109.588) (end 164.592 111.7191) (width 0.1524) (layer F.Cu) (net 14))
 (segment (start 164.592 109.22) (end 164.592 109.243) (width 0.1524) (layer F.Cu) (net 14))
 (segment (start 164.592 109.243) (end 164.592 109.588) (width 0.1524) (layer F.Cu) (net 14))
 (segment (start 190.8559 122.9995) (end 190.7924 122.936) (width 0.1524) (layer F.Cu) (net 14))
 (segment (start 194.8233 122.9995) (end 190.8559 122.9995) (width 0.1524) (layer F.Cu) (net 14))
 (segment (start 196.0669 121.7559) (end 194.8233 122.9995) (width 0.1524) (layer F.Cu) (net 14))
 (segment (start 196.0669 100.378) (end 196.0669 121.7559) (width 0.1524) (layer F.Cu) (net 14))
 (segment (start 195.5114 99.8225) (end 196.0669 100.378) (width 0.1524) (layer F.Cu) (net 14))
 (segment (start 186.1792 99.8225) (end 195.5114 99.8225) (width 0.1524) (layer F.Cu) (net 14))
 (segment (start 185.5885 100.4132) (end 186.1792 99.8225) (width 0.1524) (layer F.Cu) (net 14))
 (segment (start 185.5885 101.2363) (end 185.5885 100.4132) (width 0.1524) (layer F.Cu) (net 14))
 (segment (start 182.6475 104.1773) (end 185.5885 101.2363) (width 0.1524) (layer F.Cu) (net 14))
 (segment (start 169.6577 104.1773) (end 182.6475 104.1773) (width 0.1524) (layer F.Cu) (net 14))
 (segment (start 164.592 109.243) (end 169.6577 104.1773) (width 0.1524) (layer F.Cu) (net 14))
 (segment (start 189.992 122.936) (end 190.7924 122.936) (width 0.1524) (layer F.Cu) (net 14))
 (segment (start 166.5411 116.84) (end 165.862 116.84) (width 0.1524) (layer F.Cu) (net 17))
 (segment (start 166.7011 117) (end 166.5411 116.84) (width 0.1524) (layer F.Cu) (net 17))
 (segment (start 168.88 117) (end 166.7011 117) (width 0.1524) (layer F.Cu) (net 17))
 (segment (start 187.452 127) (end 187.452 123.19) (width 0.1524) (layer F.Cu) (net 2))
 (segment (start 186.436 125.984) (end 187.452 127) (width 0.1524) (layer F.Cu) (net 2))
 (segment (start 182.372 125.984) (end 186.436 125.984) (width 0.1524) (layer F.Cu) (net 2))
 (segment (start 181.737 125.349) (end 182.372 125.984) (width 0.1524) (layer F.Cu) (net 2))
 (segment (start 181.737 113.919) (end 181.737 125.349) (width 0.1524) (layer F.Cu) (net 2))
 (segment (start 182.656 113) (end 181.737 113.919) (width 0.1524) (layer F.Cu) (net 2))
 (segment (start 182.88 113) (end 182.656 113) (width 0.1524) (layer F.Cu) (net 2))
 (segment (start 187.452 107.442) (end 185.42 107.442) (width 0.3048) (layer F.Cu) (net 2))
 (segment (start 190.754 104.14) (end 187.452 107.442) (width 0.3048) (layer F.Cu) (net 2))
 (segment (start 194.31 104.14) (end 190.754 104.14) (width 0.3048) (layer F.Cu) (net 2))
 (segment (start 182.89 107.442) (end 182.88 107.432) (width 0.3048) (layer F.Cu) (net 2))
 (segment (start 185.42 107.442) (end 182.89 107.442) (width 0.3048) (layer F.Cu) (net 2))
 (segment (start 182.88 107.432) (end 182.88 107.4318) (width 0.1524) (layer F.Cu) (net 2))
 (segment (start 180.975 106.299) (end 179.705 105.029) (width 0.1524) (layer F.Cu) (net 2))
 (segment (start 180.975 106.426) (end 180.975 106.299) (width 0.1524) (layer F.Cu) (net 2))
 (segment (start 181.981 107.432) (end 180.975 106.426) (width 0.1524) (layer F.Cu) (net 2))
 (segment (start 182.88 107.432) (end 181.981 107.432) (width 0.1524) (layer F.Cu) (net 2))
 (segment (start 182.88 107.432) (end 182.88 109.9698) (width 0.3048) (layer F.Cu) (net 2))
 (segment (start 182.88 109.9698) (end 182.88 113) (width 0.3048) (layer F.Cu) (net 2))
 (segment (start 164.338 118.745) (end 164.338 116.84) (width 0.1524) (layer F.Cu) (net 2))
 (segment (start 164.338 116.84) (end 164.338 116.0396) (width 0.1524) (layer F.Cu) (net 2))
 (segment (start 168.032 109.9698) (end 182.88 109.9698) (width 0.1524) (layer F.Cu) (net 2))
 (segment (start 163.7915 114.2103) (end 168.032 109.9698) (width 0.1524) (layer F.Cu) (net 2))
 (segment (start 163.7915 115.6283) (end 163.7915 114.2103) (width 0.1524) (layer F.Cu) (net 2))
 (segment (start 164.2028 116.0396) (end 163.7915 115.6283) (width 0.1524) (layer F.Cu) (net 2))
 (segment (start 164.338 116.0396) (end 164.2028 116.0396) (width 0.1524) (layer F.Cu) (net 2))
 (segment (start 164.338 125.095) (end 163.7916 125.095) (width 0.1524) (layer F.Cu) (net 11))
 (segment (start 183.27 100.965) (end 183.27 102.0689) (width 0.1524) (layer F.Cu) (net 11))
 (segment (start 158.75 128.515) (end 159.8539 128.515) (width 0.1524) (layer F.Cu) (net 11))
 (segment (start 159.8539 128.515) (end 163.3441 125.0248) (width 0.1524) (layer F.Cu) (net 11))
 (segment (start 163.4142 125.095) (end 163.7916 125.095) (width 0.1524) (layer F.Cu) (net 11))
 (segment (start 163.3441 125.0248) (end 163.4142 125.095) (width 0.1524) (layer F.Cu) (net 11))
 (segment (start 163.1358 124.8166) (end 163.3441 125.0248) (width 0.1524) (layer F.Cu) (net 11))
 (segment (start 163.1358 121.4181) (end 163.1358 124.8166) (width 0.1524) (layer F.Cu) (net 11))
 (segment (start 162.8307 121.113) (end 163.1358 121.4181) (width 0.1524) (layer F.Cu) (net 11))
 (segment (start 162.8307 120.2412) (end 162.8307 121.113) (width 0.1524) (layer F.Cu) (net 11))
 (segment (start 162.6781 120.0886) (end 162.8307 120.2412) (width 0.1524) (layer F.Cu) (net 11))
 (segment (start 162.6781 119.9688) (end 162.6781 120.0886) (width 0.1524) (layer F.Cu) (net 11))
 (segment (start 162.5256 119.8163) (end 162.6781 119.9688) (width 0.1524) (layer F.Cu) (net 11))
 (segment (start 162.5256 112.8865) (end 162.5256 119.8163) (width 0.1524) (layer F.Cu) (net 11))
 (segment (start 162.5515 112.8606) (end 162.5256 112.8865) (width 0.1524) (layer F.Cu) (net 11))
 (segment (start 162.5515 112.5914) (end 162.5515 112.8606) (width 0.1524) (layer F.Cu) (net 11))
 (segment (start 163.4166 111.7263) (end 162.5515 112.5914) (width 0.1524) (layer F.Cu) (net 11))
 (segment (start 163.4166 110.6594) (end 163.4166 111.7263) (width 0.1524) (layer F.Cu) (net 11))
 (segment (start 163.6958 110.3802) (end 163.4166 110.6594) (width 0.1524) (layer F.Cu) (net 11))
 (segment (start 163.6958 110.1643) (end 163.6958 110.3802) (width 0.1524) (layer F.Cu) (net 11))
 (segment (start 164.0009 109.8592) (end 163.6958 110.1643) (width 0.1524) (layer F.Cu) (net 11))
 (segment (start 164.0009 108.5516) (end 164.0009 109.8592) (width 0.1524) (layer F.Cu) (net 11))
 (segment (start 169.0601 103.4924) (end 164.0009 108.5516) (width 0.1524) (layer F.Cu) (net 11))
 (segment (start 178.295 103.4924) (end 169.0601 103.4924) (width 0.1524) (layer F.Cu) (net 11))
 (segment (start 178.5253 103.2621) (end 178.295 103.4924) (width 0.1524) (layer F.Cu) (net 11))
 (segment (start 179.5996 103.2621) (end 178.5253 103.2621) (width 0.1524) (layer F.Cu) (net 11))
 (segment (start 179.9047 102.957) (end 179.5996 103.2621) (width 0.1524) (layer F.Cu) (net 11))
 (segment (start 181.284 102.957) (end 179.9047 102.957) (width 0.1524) (layer F.Cu) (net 11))
 (segment (start 181.2841 102.9569) (end 181.284 102.957) (width 0.1524) (layer F.Cu) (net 11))
 (segment (start 181.9504 102.9569) (end 181.2841 102.9569) (width 0.1524) (layer F.Cu) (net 11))
 (segment (start 182.1725 102.7348) (end 181.9504 102.9569) (width 0.1524) (layer F.Cu) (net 11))
 (segment (start 182.6041 102.7348) (end 182.1725 102.7348) (width 0.1524) (layer F.Cu) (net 11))
 (segment (start 183.27 102.0689) (end 182.6041 102.7348) (width 0.1524) (layer F.Cu) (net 11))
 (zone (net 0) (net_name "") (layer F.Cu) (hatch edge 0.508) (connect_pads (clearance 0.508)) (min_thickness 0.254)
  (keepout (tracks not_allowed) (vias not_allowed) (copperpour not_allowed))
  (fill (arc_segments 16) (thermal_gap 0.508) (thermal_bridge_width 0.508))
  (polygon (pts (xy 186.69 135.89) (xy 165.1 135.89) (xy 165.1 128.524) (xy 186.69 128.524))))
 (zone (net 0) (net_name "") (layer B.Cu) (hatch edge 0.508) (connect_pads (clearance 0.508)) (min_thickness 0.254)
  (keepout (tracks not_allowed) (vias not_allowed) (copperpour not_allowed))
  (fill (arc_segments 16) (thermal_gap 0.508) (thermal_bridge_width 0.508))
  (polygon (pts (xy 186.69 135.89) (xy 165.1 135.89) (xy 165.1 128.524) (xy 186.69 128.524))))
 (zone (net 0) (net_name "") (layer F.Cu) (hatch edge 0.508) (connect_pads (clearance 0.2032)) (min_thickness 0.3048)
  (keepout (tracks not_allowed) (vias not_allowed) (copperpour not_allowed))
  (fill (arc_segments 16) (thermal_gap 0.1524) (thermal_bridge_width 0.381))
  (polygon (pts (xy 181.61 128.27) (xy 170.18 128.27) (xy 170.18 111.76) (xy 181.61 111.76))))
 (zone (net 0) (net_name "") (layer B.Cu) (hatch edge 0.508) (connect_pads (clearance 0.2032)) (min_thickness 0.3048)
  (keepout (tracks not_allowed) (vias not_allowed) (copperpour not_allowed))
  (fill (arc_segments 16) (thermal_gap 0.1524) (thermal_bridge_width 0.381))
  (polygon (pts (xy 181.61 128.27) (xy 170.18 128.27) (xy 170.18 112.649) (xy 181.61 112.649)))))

